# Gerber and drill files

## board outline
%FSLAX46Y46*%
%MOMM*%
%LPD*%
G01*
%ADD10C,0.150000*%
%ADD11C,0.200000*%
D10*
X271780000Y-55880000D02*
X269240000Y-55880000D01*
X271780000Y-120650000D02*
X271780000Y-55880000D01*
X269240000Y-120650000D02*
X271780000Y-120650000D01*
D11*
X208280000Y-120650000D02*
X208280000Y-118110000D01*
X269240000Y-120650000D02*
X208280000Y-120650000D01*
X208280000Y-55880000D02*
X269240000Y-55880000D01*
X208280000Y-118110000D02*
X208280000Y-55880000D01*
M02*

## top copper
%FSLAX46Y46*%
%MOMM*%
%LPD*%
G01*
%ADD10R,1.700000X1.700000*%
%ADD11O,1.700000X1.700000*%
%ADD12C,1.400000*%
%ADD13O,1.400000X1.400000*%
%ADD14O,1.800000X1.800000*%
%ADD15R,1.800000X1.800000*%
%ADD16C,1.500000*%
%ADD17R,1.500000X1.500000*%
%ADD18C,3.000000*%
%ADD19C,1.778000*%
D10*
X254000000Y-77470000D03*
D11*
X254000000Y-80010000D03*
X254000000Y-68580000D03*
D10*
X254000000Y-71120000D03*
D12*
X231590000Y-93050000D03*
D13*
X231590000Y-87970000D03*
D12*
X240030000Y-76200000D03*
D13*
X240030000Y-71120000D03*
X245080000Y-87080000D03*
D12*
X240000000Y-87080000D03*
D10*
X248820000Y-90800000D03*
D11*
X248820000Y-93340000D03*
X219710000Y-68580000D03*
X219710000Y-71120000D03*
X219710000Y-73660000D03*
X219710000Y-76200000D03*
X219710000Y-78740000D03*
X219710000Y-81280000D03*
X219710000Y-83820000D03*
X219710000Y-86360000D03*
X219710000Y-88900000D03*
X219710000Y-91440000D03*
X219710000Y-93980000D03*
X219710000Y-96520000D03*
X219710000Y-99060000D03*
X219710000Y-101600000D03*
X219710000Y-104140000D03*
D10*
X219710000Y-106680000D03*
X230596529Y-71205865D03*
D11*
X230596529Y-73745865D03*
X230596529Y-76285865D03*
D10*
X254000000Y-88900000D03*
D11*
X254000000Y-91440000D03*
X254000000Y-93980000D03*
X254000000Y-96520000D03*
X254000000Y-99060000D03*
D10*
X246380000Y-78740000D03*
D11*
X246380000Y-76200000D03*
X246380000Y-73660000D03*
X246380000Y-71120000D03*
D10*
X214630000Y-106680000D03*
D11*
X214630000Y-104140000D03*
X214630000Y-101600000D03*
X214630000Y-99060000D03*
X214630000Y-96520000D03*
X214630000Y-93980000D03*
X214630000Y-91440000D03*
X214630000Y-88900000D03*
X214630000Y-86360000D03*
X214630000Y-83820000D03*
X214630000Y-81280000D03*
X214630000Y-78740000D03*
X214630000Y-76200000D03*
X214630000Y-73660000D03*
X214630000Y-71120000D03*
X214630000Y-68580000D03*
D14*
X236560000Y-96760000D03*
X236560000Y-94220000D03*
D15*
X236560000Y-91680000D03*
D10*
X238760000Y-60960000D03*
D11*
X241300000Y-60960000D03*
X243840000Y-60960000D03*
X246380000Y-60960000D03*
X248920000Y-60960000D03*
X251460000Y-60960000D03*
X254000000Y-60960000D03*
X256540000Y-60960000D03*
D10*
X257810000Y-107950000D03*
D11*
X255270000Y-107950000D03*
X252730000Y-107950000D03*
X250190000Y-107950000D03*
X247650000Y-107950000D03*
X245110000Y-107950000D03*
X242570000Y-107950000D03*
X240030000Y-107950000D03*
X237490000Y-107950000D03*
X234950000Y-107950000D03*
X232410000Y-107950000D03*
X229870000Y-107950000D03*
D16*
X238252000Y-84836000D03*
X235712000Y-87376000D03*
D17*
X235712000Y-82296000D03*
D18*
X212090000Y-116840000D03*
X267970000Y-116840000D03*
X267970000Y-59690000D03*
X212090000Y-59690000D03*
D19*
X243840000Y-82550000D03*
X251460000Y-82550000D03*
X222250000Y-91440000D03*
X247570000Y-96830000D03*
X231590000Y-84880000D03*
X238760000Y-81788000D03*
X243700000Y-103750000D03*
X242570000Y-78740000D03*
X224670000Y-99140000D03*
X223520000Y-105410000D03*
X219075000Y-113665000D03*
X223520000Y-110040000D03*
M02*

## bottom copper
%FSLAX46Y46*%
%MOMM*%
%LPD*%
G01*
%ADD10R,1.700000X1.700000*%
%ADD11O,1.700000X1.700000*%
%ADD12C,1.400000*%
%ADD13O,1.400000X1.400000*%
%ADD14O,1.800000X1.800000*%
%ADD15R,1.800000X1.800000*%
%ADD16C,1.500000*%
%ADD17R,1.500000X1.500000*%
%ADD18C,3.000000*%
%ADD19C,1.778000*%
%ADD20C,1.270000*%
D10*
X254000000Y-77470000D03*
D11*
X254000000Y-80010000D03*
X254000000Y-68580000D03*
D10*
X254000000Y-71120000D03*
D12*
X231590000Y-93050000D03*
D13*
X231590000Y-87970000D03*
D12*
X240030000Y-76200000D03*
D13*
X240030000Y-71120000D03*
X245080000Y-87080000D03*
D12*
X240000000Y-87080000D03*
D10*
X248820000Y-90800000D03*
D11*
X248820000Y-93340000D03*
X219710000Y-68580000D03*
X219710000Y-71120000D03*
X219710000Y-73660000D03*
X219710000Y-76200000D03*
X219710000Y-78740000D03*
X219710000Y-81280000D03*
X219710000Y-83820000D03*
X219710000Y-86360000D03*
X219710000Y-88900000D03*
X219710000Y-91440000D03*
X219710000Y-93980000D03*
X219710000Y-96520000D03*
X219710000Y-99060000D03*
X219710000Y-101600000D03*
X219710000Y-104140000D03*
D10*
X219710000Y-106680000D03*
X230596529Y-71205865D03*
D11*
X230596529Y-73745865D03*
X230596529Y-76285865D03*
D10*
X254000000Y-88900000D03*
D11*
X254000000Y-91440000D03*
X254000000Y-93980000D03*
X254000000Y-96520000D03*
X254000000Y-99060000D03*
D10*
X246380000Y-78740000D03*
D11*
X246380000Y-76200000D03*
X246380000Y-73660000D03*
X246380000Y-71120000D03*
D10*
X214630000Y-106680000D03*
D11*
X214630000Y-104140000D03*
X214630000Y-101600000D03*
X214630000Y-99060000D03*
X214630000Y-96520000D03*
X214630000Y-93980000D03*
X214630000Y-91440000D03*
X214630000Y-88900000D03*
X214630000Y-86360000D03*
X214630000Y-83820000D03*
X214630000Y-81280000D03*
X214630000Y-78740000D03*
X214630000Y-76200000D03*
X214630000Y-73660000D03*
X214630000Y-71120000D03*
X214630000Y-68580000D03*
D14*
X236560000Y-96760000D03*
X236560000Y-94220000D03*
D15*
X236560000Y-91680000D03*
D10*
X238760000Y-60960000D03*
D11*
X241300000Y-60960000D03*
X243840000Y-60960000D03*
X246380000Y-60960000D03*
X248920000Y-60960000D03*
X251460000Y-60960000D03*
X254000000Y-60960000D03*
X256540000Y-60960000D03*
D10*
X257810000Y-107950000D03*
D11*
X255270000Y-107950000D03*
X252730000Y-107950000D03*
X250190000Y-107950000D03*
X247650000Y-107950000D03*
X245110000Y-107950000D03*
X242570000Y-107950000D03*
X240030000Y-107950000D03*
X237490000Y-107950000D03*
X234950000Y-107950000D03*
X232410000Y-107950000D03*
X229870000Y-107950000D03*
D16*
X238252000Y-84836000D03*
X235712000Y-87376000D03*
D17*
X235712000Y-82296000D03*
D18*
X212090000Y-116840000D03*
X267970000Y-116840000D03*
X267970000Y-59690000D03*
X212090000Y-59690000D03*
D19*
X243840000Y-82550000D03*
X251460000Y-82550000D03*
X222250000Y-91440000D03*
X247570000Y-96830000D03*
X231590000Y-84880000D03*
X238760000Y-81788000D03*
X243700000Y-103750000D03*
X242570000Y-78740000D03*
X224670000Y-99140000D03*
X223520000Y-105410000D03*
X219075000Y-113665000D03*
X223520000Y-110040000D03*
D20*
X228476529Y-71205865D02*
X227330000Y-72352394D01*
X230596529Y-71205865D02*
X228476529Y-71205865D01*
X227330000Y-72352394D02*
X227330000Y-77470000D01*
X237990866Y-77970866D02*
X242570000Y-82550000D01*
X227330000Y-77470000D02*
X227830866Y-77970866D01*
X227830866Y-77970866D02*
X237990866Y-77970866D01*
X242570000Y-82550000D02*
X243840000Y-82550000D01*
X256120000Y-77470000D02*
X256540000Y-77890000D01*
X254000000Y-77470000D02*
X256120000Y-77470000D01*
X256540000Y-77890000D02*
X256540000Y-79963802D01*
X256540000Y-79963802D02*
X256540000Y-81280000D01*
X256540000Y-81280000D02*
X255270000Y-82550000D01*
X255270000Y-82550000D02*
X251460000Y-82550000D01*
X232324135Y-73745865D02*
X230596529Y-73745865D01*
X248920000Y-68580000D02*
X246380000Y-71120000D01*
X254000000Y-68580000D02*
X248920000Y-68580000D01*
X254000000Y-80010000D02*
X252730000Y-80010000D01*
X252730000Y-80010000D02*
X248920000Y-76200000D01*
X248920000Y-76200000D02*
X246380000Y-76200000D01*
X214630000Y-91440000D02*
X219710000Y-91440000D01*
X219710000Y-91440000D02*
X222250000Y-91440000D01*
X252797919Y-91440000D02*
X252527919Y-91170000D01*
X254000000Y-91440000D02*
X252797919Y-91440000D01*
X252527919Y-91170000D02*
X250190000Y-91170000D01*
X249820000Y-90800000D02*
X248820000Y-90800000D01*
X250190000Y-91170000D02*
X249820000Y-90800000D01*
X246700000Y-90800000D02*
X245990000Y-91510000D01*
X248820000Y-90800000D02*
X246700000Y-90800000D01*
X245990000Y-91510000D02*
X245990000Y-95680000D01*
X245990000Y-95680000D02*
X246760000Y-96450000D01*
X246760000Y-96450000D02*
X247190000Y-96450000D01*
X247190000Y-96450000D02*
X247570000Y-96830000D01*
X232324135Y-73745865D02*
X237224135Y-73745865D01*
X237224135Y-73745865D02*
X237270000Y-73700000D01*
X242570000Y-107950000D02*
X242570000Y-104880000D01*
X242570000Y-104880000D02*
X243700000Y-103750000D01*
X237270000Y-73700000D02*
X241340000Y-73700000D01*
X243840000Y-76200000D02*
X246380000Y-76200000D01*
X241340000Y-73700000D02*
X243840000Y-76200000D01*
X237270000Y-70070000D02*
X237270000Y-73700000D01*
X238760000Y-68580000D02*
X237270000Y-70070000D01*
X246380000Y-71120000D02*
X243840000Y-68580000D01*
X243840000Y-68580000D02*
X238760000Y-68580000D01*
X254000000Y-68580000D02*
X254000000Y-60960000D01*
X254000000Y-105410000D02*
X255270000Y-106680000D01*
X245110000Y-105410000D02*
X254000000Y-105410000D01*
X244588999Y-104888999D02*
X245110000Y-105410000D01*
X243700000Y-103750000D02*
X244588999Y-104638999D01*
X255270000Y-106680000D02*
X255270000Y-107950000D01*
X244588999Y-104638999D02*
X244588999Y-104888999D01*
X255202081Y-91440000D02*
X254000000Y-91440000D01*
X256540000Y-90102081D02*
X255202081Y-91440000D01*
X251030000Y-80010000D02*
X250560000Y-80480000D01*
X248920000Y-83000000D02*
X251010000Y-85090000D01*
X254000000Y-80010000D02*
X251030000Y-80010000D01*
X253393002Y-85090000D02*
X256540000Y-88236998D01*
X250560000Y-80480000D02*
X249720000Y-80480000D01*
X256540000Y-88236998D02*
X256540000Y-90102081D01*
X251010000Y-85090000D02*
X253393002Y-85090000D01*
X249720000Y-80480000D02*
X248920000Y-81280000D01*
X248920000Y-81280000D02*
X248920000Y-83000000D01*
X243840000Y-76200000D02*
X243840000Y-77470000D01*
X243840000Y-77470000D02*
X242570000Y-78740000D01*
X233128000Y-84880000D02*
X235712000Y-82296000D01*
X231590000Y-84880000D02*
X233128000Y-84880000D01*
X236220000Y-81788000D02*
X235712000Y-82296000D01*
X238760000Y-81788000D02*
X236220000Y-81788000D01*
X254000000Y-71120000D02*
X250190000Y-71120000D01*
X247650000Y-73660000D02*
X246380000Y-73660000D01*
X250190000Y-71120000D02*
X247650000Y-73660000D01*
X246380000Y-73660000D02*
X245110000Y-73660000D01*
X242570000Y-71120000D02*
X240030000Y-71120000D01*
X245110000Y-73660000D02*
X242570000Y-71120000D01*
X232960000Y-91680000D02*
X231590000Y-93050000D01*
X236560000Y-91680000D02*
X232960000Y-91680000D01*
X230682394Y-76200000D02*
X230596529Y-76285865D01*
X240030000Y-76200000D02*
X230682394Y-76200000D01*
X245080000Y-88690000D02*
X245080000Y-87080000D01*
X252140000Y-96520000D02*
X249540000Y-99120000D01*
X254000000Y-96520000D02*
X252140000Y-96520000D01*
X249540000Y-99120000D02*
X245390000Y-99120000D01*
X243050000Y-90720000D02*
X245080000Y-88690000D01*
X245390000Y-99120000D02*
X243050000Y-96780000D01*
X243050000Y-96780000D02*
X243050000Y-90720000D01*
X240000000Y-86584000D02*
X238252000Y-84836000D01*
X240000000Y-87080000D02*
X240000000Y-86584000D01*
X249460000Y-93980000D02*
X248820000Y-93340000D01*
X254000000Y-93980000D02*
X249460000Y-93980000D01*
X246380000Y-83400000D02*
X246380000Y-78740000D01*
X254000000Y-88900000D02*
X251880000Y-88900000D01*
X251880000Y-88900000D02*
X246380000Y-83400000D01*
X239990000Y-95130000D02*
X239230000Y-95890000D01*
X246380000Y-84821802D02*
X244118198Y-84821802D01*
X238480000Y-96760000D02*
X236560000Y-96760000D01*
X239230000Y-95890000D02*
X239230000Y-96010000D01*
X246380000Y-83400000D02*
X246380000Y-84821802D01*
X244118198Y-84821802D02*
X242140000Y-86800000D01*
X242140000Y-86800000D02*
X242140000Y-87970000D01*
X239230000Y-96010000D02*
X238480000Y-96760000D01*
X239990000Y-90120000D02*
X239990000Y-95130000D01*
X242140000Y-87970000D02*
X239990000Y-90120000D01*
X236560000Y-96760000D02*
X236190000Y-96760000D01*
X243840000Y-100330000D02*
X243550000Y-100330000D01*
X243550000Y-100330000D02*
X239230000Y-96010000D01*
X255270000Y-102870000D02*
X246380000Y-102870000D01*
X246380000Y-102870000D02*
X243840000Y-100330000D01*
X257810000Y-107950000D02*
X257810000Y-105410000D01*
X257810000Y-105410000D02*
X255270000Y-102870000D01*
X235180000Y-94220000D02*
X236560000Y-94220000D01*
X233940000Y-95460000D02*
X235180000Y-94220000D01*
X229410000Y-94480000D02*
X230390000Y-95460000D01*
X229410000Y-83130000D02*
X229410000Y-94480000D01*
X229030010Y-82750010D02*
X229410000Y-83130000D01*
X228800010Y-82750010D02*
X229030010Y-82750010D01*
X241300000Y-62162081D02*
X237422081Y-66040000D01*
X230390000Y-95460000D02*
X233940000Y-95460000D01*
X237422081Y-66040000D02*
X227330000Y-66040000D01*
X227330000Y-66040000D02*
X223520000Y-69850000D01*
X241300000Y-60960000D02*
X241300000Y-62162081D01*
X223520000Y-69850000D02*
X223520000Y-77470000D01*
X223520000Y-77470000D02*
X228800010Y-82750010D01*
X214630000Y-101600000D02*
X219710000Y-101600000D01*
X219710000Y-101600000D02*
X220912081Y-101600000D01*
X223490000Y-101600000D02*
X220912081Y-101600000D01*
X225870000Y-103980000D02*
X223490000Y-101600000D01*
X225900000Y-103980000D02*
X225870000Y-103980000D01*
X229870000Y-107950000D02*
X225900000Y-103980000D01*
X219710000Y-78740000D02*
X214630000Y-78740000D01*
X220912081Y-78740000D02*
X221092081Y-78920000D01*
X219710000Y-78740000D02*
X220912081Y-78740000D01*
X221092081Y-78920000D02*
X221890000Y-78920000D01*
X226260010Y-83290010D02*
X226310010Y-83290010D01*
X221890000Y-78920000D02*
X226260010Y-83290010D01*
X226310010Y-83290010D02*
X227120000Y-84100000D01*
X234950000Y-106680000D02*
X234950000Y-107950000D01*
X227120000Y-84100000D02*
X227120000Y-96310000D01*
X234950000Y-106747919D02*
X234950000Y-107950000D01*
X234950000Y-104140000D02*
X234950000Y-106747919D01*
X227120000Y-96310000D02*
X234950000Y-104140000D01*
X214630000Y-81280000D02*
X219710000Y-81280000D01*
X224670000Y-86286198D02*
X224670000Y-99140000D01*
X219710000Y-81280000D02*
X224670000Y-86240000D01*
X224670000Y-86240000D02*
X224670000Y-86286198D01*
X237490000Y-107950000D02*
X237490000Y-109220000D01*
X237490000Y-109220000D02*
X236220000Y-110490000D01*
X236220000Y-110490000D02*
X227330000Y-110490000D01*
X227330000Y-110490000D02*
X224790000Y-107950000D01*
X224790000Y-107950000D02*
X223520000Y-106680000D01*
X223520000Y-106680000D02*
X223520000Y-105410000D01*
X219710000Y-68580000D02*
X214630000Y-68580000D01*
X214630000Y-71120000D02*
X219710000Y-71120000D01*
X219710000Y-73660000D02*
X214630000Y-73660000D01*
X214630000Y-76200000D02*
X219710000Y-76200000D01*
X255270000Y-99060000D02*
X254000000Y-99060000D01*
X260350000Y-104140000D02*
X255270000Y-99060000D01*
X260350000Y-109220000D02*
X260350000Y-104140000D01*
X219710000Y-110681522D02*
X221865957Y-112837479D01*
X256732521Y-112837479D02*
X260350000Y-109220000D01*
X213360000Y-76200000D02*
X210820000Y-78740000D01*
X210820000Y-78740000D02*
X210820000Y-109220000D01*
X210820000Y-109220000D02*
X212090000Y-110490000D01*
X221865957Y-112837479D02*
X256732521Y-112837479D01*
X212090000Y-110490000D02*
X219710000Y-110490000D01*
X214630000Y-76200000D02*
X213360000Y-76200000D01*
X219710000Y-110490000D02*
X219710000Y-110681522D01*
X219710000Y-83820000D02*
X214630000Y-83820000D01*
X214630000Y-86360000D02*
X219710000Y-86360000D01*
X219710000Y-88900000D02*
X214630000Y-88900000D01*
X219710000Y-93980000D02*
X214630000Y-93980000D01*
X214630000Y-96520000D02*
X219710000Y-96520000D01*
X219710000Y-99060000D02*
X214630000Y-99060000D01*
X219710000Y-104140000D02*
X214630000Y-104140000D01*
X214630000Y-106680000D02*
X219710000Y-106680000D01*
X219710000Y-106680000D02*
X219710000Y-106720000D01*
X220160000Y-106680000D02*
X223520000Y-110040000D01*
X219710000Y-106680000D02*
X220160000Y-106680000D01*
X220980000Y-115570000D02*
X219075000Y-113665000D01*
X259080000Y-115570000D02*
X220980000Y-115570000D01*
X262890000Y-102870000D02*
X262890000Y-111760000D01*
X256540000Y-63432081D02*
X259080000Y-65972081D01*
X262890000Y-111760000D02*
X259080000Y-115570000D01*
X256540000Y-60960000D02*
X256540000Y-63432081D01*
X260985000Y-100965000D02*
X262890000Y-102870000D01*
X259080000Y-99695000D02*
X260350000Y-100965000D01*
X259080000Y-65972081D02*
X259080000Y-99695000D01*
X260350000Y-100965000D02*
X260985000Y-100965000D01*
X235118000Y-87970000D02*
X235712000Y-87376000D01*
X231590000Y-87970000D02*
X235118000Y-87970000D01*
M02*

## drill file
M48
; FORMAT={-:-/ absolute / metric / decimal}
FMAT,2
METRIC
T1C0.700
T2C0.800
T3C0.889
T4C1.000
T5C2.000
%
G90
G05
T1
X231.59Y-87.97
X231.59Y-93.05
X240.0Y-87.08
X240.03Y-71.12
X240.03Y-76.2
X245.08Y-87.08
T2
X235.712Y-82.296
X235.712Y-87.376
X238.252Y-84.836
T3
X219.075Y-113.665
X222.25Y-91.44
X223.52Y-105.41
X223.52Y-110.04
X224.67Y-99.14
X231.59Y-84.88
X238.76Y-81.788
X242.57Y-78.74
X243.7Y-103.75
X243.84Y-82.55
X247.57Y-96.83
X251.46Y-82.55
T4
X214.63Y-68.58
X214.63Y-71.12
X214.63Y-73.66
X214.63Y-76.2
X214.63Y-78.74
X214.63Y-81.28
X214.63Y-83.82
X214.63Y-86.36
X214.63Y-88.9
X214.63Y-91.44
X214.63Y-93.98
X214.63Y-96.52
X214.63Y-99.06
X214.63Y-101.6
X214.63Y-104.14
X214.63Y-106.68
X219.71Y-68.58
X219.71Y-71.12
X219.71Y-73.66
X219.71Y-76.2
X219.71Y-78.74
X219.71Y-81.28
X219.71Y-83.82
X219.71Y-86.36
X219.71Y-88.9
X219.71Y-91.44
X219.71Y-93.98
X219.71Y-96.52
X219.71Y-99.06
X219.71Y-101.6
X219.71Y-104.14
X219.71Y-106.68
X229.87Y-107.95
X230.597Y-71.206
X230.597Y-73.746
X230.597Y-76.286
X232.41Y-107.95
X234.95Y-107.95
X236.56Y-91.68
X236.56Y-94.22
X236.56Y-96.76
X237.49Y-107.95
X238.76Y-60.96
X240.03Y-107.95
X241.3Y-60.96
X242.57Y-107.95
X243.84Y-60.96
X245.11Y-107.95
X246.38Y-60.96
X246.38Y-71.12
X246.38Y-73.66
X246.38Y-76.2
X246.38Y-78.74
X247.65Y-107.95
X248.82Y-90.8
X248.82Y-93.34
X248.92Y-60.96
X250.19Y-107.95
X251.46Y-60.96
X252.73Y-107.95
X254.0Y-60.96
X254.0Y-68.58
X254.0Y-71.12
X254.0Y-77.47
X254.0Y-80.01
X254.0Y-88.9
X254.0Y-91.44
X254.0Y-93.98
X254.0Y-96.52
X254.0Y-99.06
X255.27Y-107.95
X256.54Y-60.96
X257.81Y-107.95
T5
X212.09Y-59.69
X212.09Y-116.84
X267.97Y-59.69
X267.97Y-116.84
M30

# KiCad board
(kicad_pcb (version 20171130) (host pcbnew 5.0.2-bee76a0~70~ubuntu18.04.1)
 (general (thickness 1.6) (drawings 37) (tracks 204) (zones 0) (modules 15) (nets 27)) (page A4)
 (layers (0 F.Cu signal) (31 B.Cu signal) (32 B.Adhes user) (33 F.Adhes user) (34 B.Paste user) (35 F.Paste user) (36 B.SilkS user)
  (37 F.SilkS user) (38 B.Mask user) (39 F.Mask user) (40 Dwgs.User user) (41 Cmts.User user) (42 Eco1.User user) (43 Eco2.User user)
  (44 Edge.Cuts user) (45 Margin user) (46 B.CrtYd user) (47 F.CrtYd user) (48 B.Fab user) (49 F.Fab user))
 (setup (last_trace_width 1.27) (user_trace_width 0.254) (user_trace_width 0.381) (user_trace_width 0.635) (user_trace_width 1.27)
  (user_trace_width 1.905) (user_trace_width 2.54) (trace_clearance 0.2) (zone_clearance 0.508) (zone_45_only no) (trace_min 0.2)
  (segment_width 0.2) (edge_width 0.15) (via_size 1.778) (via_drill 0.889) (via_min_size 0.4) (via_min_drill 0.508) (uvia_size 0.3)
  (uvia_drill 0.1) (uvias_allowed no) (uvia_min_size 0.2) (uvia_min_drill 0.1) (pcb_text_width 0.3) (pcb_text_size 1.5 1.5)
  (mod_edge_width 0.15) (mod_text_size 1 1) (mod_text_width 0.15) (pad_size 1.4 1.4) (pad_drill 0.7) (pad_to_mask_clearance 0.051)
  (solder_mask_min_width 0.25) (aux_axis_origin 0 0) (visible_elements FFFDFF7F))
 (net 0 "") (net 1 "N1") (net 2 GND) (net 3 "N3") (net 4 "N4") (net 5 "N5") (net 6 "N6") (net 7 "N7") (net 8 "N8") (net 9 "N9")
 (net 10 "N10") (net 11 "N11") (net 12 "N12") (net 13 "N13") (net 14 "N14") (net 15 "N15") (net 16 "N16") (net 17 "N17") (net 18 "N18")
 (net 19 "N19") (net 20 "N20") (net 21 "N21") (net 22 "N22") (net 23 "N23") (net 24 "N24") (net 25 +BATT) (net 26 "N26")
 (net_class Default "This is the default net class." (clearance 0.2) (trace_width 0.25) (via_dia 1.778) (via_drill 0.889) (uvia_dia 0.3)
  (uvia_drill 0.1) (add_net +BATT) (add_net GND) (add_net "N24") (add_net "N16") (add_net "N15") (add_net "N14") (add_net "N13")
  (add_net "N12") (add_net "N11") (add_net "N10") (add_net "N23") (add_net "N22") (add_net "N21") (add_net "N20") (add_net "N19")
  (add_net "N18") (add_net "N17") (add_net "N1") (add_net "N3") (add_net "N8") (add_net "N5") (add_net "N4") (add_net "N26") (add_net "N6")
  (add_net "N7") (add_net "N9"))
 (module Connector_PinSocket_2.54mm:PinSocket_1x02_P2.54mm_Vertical (layer F.Cu) (at 254 77.47)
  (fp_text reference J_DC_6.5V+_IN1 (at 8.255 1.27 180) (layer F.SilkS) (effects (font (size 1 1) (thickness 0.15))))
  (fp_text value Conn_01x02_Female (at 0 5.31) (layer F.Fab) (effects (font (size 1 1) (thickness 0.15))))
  (pad 1 thru_hole rect (at 0 0) (size 1.7 1.7) (drill 1) (layers *.Cu *.Mask) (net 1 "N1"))
  (pad 2 thru_hole oval (at 0 2.54) (size 1.7 1.7) (drill 1) (layers *.Cu *.Mask) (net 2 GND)))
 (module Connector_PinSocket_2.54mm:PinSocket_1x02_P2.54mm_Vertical (layer F.Cu) (at 254 71.12 180)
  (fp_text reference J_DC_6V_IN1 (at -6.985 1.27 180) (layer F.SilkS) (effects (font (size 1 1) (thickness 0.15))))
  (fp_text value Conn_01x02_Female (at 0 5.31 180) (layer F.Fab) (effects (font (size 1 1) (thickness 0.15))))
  (pad 2 thru_hole oval (at 0 2.54 180) (size 1.7 1.7) (drill 1) (layers *.Cu *.Mask) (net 2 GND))
  (pad 1 thru_hole rect (at 0 0 180) (size 1.7 1.7) (drill 1) (layers *.Cu *.Mask) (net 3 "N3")))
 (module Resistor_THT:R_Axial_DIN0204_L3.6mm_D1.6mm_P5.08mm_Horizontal (layer F.Cu) (at 231.59 93.05 90)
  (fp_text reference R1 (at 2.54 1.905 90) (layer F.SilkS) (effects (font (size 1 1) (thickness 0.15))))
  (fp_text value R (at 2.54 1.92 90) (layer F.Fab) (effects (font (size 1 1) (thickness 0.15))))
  (pad 1 thru_hole circle (at 0 0 90) (size 1.4 1.4) (drill 0.7) (layers *.Cu *.Mask) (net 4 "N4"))
  (pad 2 thru_hole oval (at 5.08 0 90) (size 1.4 1.4) (drill 0.7) (layers *.Cu *.Mask) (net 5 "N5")))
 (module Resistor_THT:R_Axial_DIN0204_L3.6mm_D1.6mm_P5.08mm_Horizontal (layer F.Cu) (at 240.03 76.2 90)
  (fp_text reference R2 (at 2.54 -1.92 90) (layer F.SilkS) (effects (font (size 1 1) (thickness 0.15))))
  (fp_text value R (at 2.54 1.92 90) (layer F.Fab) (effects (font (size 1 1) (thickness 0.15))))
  (pad 1 thru_hole circle (at 0 0 90) (size 1.4 1.4) (drill 0.7) (layers *.Cu *.Mask) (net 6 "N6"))
  (pad 2 thru_hole oval (at 5.08 0 90) (size 1.4 1.4) (drill 0.7) (layers *.Cu *.Mask) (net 3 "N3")))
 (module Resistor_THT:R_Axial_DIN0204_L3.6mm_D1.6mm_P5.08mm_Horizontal (layer F.Cu) (at 240 87.08)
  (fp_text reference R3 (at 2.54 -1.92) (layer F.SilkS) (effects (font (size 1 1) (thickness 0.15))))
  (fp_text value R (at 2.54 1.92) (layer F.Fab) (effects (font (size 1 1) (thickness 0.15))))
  (pad 2 thru_hole oval (at 5.08 0) (size 1.4 1.4) (drill 0.7) (layers *.Cu *.Mask) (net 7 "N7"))
  (pad 1 thru_hole circle (at 0 0) (size 1.4 1.4) (drill 0.7) (layers *.Cu *.Mask) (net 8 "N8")))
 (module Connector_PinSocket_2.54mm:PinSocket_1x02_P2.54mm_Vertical (layer F.Cu) (at 248.82 90.8)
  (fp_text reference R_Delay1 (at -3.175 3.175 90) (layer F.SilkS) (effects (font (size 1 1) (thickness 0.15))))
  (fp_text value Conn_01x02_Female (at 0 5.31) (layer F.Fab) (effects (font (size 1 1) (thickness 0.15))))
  (pad 1 thru_hole rect (at 0 0) (size 1.7 1.7) (drill 1) (layers *.Cu *.Mask) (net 2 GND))
  (pad 2 thru_hole oval (at 0 2.54) (size 1.7 1.7) (drill 1) (layers *.Cu *.Mask) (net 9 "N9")))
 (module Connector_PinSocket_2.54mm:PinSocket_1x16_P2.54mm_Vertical (layer F.Cu) (at 219.71 106.68 180)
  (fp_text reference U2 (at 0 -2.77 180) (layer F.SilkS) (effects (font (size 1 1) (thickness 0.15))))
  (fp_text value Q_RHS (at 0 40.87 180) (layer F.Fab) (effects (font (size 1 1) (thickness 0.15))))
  (pad 16 thru_hole oval (at 0 38.1 180) (size 1.7 1.7) (drill 1) (layers *.Cu *.Mask) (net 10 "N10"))
  (pad 15 thru_hole oval (at 0 35.56 180) (size 1.7 1.7) (drill 1) (layers *.Cu *.Mask) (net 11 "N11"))
  (pad 14 thru_hole oval (at 0 33.02 180) (size 1.7 1.7) (drill 1) (layers *.Cu *.Mask) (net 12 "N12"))
  (pad 13 thru_hole oval (at 0 30.48 180) (size 1.7 1.7) (drill 1) (layers *.Cu *.Mask) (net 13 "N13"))
  (pad 12 thru_hole oval (at 0 27.94 180) (size 1.7 1.7) (drill 1) (layers *.Cu *.Mask) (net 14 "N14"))
  (pad 11 thru_hole oval (at 0 25.4 180) (size 1.7 1.7) (drill 1) (layers *.Cu *.Mask) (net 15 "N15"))
  (pad 10 thru_hole oval (at 0 22.86 180) (size 1.7 1.7) (drill 1) (layers *.Cu *.Mask) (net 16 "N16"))
  (pad 9 thru_hole oval (at 0 20.32 180) (size 1.7 1.7) (drill 1) (layers *.Cu *.Mask) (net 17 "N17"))
  (pad 8 thru_hole oval (at 0 17.78 180) (size 1.7 1.7) (drill 1) (layers *.Cu *.Mask) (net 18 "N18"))
  (pad 7 thru_hole oval (at 0 15.24 180) (size 1.7 1.7) (drill 1) (layers *.Cu *.Mask) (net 2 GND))
  (pad 6 thru_hole oval (at 0 12.7 180) (size 1.7 1.7) (drill 1) (layers *.Cu *.Mask) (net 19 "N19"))
  (pad 5 thru_hole oval (at 0 10.16 180) (size 1.7 1.7) (drill 1) (layers *.Cu *.Mask) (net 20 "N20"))
  (pad 4 thru_hole oval (at 0 7.62 180) (size 1.7 1.7) (drill 1) (layers *.Cu *.Mask) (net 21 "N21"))
  (pad 3 thru_hole oval (at 0 5.08 180) (size 1.7 1.7) (drill 1) (layers *.Cu *.Mask) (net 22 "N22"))
  (pad 2 thru_hole oval (at 0 2.54 180) (size 1.7 1.7) (drill 1) (layers *.Cu *.Mask) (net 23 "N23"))
  (pad 1 thru_hole rect (at 0 0 180) (size 1.7 1.7) (drill 1) (layers *.Cu *.Mask) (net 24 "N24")))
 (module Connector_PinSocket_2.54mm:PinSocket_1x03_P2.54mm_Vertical (layer F.Cu) (at 230.596529 71.205865)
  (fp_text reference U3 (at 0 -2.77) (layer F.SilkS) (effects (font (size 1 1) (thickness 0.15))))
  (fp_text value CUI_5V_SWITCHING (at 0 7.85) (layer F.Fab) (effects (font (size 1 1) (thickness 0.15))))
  (pad 1 thru_hole rect (at 0 0) (size 1.7 1.7) (drill 1) (layers *.Cu *.Mask) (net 1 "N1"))
  (pad 2 thru_hole oval (at 0 2.54) (size 1.7 1.7) (drill 1) (layers *.Cu *.Mask) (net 2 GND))
  (pad 3 thru_hole oval (at 0 5.08) (size 1.7 1.7) (drill 1) (layers *.Cu *.Mask) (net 6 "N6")))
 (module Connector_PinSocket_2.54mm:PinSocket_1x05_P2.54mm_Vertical (layer F.Cu) (at 254 88.9)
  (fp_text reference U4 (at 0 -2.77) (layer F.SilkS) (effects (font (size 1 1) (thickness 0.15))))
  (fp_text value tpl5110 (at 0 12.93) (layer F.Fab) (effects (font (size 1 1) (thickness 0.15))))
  (pad 1 thru_hole rect (at 0 0) (size 1.7 1.7) (drill 1) (layers *.Cu *.Mask) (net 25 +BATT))
  (pad 2 thru_hole oval (at 0 2.54) (size 1.7 1.7) (drill 1) (layers *.Cu *.Mask) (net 2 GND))
  (pad 3 thru_hole oval (at 0 5.08) (size 1.7 1.7) (drill 1) (layers *.Cu *.Mask) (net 9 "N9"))
  (pad 4 thru_hole oval (at 0 7.62) (size 1.7 1.7) (drill 1) (layers *.Cu *.Mask) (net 7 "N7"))
  (pad 5 thru_hole oval (at 0 10.16) (size 1.7 1.7) (drill 1) (layers *.Cu *.Mask) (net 13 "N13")))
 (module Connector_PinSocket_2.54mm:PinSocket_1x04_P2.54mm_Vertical (layer F.Cu) (at 246.38 78.74 180)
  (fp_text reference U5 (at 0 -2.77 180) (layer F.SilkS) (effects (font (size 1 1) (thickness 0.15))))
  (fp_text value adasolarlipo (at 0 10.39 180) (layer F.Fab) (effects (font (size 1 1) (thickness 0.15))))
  (pad 1 thru_hole rect (at 0 0 180) (size 1.7 1.7) (drill 1) (layers *.Cu *.Mask) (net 25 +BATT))
  (pad 2 thru_hole oval (at 0 2.54 180) (size 1.7 1.7) (drill 1) (layers *.Cu *.Mask) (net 2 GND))
  (pad 3 thru_hole oval (at 0 5.08 180) (size 1.7 1.7) (drill 1) (layers *.Cu *.Mask) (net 3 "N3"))
  (pad 4 thru_hole oval (at 0 7.62 180) (size 1.7 1.7) (drill 1) (layers *.Cu *.Mask) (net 2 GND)))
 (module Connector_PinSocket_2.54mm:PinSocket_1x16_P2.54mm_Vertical (layer F.Cu) (at 214.63 106.68 180)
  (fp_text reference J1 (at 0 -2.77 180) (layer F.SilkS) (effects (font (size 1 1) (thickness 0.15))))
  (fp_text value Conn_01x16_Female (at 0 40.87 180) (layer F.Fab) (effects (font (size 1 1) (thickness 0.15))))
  (pad 1 thru_hole rect (at 0 0 180) (size 1.7 1.7) (drill 1) (layers *.Cu *.Mask) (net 24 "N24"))
  (pad 2 thru_hole oval (at 0 2.54 180) (size 1.7 1.7) (drill 1) (layers *.Cu *.Mask) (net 23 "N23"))
  (pad 3 thru_hole oval (at 0 5.08 180) (size 1.7 1.7) (drill 1) (layers *.Cu *.Mask) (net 22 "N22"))
  (pad 4 thru_hole oval (at 0 7.62 180) (size 1.7 1.7) (drill 1) (layers *.Cu *.Mask) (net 21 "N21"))
  (pad 5 thru_hole oval (at 0 10.16 180) (size 1.7 1.7) (drill 1) (layers *.Cu *.Mask) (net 20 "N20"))
  (pad 6 thru_hole oval (at 0 12.7 180) (size 1.7 1.7) (drill 1) (layers *.Cu *.Mask) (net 19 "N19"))
  (pad 7 thru_hole oval (at 0 15.24 180) (size 1.7 1.7) (drill 1) (layers *.Cu *.Mask) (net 2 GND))
  (pad 8 thru_hole oval (at 0 17.78 180) (size 1.7 1.7) (drill 1) (layers *.Cu *.Mask) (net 18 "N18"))
  (pad 9 thru_hole oval (at 0 20.32 180) (size 1.7 1.7) (drill 1) (layers *.Cu *.Mask) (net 17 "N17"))
  (pad 10 thru_hole oval (at 0 22.86 180) (size 1.7 1.7) (drill 1) (layers *.Cu *.Mask) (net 16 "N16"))
  (pad 11 thru_hole oval (at 0 25.4 180) (size 1.7 1.7) (drill 1) (layers *.Cu *.Mask) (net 15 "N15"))
  (pad 12 thru_hole oval (at 0 27.94 180) (size 1.7 1.7) (drill 1) (layers *.Cu *.Mask) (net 14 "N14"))
  (pad 13 thru_hole oval (at 0 30.48 180) (size 1.7 1.7) (drill 1) (layers *.Cu *.Mask) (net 13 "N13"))
  (pad 14 thru_hole oval (at 0 33.02 180) (size 1.7 1.7) (drill 1) (layers *.Cu *.Mask) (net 12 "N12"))
  (pad 15 thru_hole oval (at 0 35.56 180) (size 1.7 1.7) (drill 1) (layers *.Cu *.Mask) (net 11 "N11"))
  (pad 16 thru_hole oval (at 0 38.1 180) (size 1.7 1.7) (drill 1) (layers *.Cu *.Mask) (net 10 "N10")))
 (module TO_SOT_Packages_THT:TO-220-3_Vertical (layer F.Cu) (at 236.56 91.68 270)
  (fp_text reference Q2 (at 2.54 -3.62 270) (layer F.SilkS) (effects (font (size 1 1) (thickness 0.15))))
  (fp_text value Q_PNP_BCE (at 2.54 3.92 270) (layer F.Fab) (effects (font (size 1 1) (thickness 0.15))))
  (pad 3 thru_hole oval (at 5.08 0 270) (size 1.8 1.8) (drill 1) (layers *.Cu *.Mask) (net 25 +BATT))
  (pad 2 thru_hole oval (at 2.54 0 270) (size 1.8 1.8) (drill 1) (layers *.Cu *.Mask) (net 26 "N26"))
  (pad 1 thru_hole rect (at 0 0 270) (size 1.8 1.8) (drill 1) (layers *.Cu *.Mask) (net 4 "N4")))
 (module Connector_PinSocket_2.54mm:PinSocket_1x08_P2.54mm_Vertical (layer F.Cu) (at 238.76 60.96 90)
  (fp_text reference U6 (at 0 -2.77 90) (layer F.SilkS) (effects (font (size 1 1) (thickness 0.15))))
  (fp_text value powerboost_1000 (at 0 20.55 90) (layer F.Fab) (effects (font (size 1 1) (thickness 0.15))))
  (pad 1 thru_hole rect (at 0 0 90) (size 1.7 1.7) (drill 1) (layers *.Cu *.Mask))
  (pad 2 thru_hole oval (at 0 2.54 90) (size 1.7 1.7) (drill 1) (layers *.Cu *.Mask) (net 26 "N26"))
  (pad 3 thru_hole oval (at 0 5.08 90) (size 1.7 1.7) (drill 1) (layers *.Cu *.Mask))
  (pad 4 thru_hole oval (at 0 7.62 90) (size 1.7 1.7) (drill 1) (layers *.Cu *.Mask))
  (pad 5 thru_hole oval (at 0 10.16 90) (size 1.7 1.7) (drill 1) (layers *.Cu *.Mask))
  (pad 6 thru_hole oval (at 0 12.7 90) (size 1.7 1.7) (drill 1) (layers *.Cu *.Mask))
  (pad 7 thru_hole oval (at 0 15.24 90) (size 1.7 1.7) (drill 1) (layers *.Cu *.Mask) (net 2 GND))
  (pad 8 thru_hole oval (at 0 17.78 90) (size 1.7 1.7) (drill 1) (layers *.Cu *.Mask) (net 24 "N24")))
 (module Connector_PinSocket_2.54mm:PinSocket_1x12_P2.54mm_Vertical (layer F.Cu) (at 257.81 107.95 270)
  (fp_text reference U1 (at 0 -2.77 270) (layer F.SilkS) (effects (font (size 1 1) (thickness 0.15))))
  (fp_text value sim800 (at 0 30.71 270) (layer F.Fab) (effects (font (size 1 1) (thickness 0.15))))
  (pad 1 thru_hole rect (at 0 0 270) (size 1.7 1.7) (drill 1) (layers *.Cu *.Mask) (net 25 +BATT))
  (pad 2 thru_hole oval (at 0 2.54 270) (size 1.7 1.7) (drill 1) (layers *.Cu *.Mask) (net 2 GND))
  (pad 3 thru_hole oval (at 0 5.08 270) (size 1.7 1.7) (drill 1) (layers *.Cu *.Mask))
  (pad 4 thru_hole oval (at 0 7.62 270) (size 1.7 1.7) (drill 1) (layers *.Cu *.Mask))
  (pad 5 thru_hole oval (at 0 10.16 270) (size 1.7 1.7) (drill 1) (layers *.Cu *.Mask))
  (pad 6 thru_hole oval (at 0 12.7 270) (size 1.7 1.7) (drill 1) (layers *.Cu *.Mask))
  (pad 7 thru_hole oval (at 0 15.24 270) (size 1.7 1.7) (drill 1) (layers *.Cu *.Mask) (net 2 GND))
  (pad 8 thru_hole oval (at 0 17.78 270) (size 1.7 1.7) (drill 1) (layers *.Cu *.Mask))
  (pad 9 thru_hole oval (at 0 20.32 270) (size 1.7 1.7) (drill 1) (layers *.Cu *.Mask) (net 15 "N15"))
  (pad 10 thru_hole oval (at 0 22.86 270) (size 1.7 1.7) (drill 1) (layers *.Cu *.Mask) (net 14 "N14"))
  (pad 11 thru_hole oval (at 0 25.4 270) (size 1.7 1.7) (drill 1) (layers *.Cu *.Mask))
  (pad 12 thru_hole oval (at 0 27.94 270) (size 1.7 1.7) (drill 1) (layers *.Cu *.Mask) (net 22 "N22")))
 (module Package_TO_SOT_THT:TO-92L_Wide (layer F.Cu) (at 235.712 82.296 270)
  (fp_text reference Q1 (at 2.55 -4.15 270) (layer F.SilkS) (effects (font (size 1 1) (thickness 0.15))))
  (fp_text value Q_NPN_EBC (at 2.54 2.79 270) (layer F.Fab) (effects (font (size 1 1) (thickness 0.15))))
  (pad 2 thru_hole circle (at 2.54 -2.54) (size 1.5 1.5) (drill 0.8) (layers *.Cu *.Mask) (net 8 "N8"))
  (pad 3 thru_hole circle (at 5.08 0) (size 1.5 1.5) (drill 0.8) (layers *.Cu *.Mask) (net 5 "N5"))
  (pad 1 thru_hole rect (at 0 0) (size 1.5 1.5) (drill 0.8) (layers *.Cu *.Mask) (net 2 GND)))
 (gr_line (start 271.78 55.88) (end 269.24 55.88) (layer Edge.Cuts) (width 0.15))
 (gr_line (start 271.78 120.65) (end 271.78 55.88) (layer Edge.Cuts) (width 0.15))
 (gr_line (start 269.24 120.65) (end 271.78 120.65) (layer Edge.Cuts) (width 0.15))
 (gr_line (start 208.28 120.65) (end 208.28 118.11) (layer Edge.Cuts) (width 0.2))
 (gr_line (start 269.24 120.65) (end 208.28 120.65) (layer Edge.Cuts) (width 0.2))
 (gr_line (start 208.28 55.88) (end 269.24 55.88) (layer Edge.Cuts) (width 0.2))
 (gr_line (start 208.28 118.11) (end 208.28 55.88) (layer Edge.Cuts) (width 0.2))
 (via (at 212.09 116.84) (size 3) (drill 2) (layers F.Cu B.Cu) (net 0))
 (via (at 267.97 116.84) (size 3) (drill 2) (layers F.Cu B.Cu) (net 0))
 (via (at 267.97 59.69) (size 3) (drill 2) (layers F.Cu B.Cu) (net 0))
 (via (at 212.09 59.69) (size 3) (drill 2) (layers F.Cu B.Cu) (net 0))
 (segment (start 228.476529 71.205865) (end 227.33 72.352394) (width 1.27) (layer B.Cu) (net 1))
 (segment (start 230.596529 71.205865) (end 228.476529 71.205865) (width 1.27) (layer B.Cu) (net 1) (status 10))
 (segment (start 227.33 72.352394) (end 227.33 77.47) (width 1.27) (layer B.Cu) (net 1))
 (segment (start 237.990866 77.970866) (end 242.57 82.55) (width 1.27) (layer B.Cu) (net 1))
 (segment (start 227.33 77.47) (end 227.830866 77.970866) (width 1.27) (layer B.Cu) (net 1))
 (segment (start 227.830866 77.970866) (end 237.990866 77.970866) (width 1.27) (layer B.Cu) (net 1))
 (via (at 243.84 82.55) (size 1.778) (drill 0.889) (layers F.Cu B.Cu) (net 1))
 (segment (start 242.57 82.55) (end 243.84 82.55) (width 1.27) (layer B.Cu) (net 1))
 (segment (start 256.12 77.47) (end 256.54 77.89) (width 1.27) (layer B.Cu) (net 1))
 (segment (start 254 77.47) (end 256.12 77.47) (width 1.27) (layer B.Cu) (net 1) (status 10))
 (segment (start 256.54 77.89) (end 256.54 79.963802) (width 1.27) (layer B.Cu) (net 1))
 (segment (start 256.54 79.963802) (end 256.54 81.28) (width 1.27) (layer B.Cu) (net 1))
 (segment (start 256.54 81.28) (end 255.27 82.55) (width 1.27) (layer B.Cu) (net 1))
 (via (at 251.46 82.55) (size 1.778) (drill 0.889) (layers F.Cu B.Cu) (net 1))
 (segment (start 255.27 82.55) (end 251.46 82.55) (width 1.27) (layer B.Cu) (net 1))
 (segment (start 232.324135 73.745865) (end 230.596529 73.745865) (width 1.27) (layer B.Cu) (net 2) (status 20))
 (segment (start 248.92 68.58) (end 246.38 71.12) (width 1.27) (layer B.Cu) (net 2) (status 20))
 (segment (start 254 68.58) (end 248.92 68.58) (width 1.27) (layer B.Cu) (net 2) (status 10))
 (segment (start 254 80.01) (end 252.73 80.01) (width 1.27) (layer B.Cu) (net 2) (status 10))
 (segment (start 252.73 80.01) (end 248.92 76.2) (width 1.27) (layer B.Cu) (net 2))
 (segment (start 248.92 76.2) (end 246.38 76.2) (width 1.27) (layer B.Cu) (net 2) (status 20))
 (segment (start 214.63 91.44) (end 219.71 91.44) (width 1.27) (layer B.Cu) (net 2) (status 30))
 (via (at 222.25 91.44) (size 1.778) (drill 0.889) (layers F.Cu B.Cu) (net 2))
 (segment (start 219.71 91.44) (end 222.25 91.44) (width 1.27) (layer B.Cu) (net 2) (status 10))
 (segment (start 252.797919 91.44) (end 252.527919 91.17) (width 1.27) (layer B.Cu) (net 2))
 (segment (start 254 91.44) (end 252.797919 91.44) (width 1.27) (layer B.Cu) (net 2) (status 10))
 (segment (start 252.527919 91.17) (end 250.19 91.17) (width 1.27) (layer B.Cu) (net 2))
 (segment (start 249.82 90.8) (end 248.82 90.8) (width 1.27) (layer B.Cu) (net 2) (status 20))
 (segment (start 250.19 91.17) (end 249.82 90.8) (width 1.27) (layer B.Cu) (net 2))
 (segment (start 246.7 90.8) (end 245.99 91.51) (width 1.27) (layer B.Cu) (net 2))
 (segment (start 248.82 90.8) (end 246.7 90.8) (width 1.27) (layer B.Cu) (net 2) (status 10))
 (segment (start 245.99 91.51) (end 245.99 95.68) (width 1.27) (layer B.Cu) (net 2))
 (segment (start 245.99 95.68) (end 246.76 96.45) (width 1.27) (layer B.Cu) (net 2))
 (via (at 247.57 96.83) (size 1.778) (drill 0.889) (layers F.Cu B.Cu) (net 2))
 (segment (start 246.76 96.45) (end 247.19 96.45) (width 1.27) (layer B.Cu) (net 2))
 (segment (start 247.19 96.45) (end 247.57 96.83) (width 1.27) (layer B.Cu) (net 2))
 (via (at 231.59 84.88) (size 1.778) (drill 0.889) (layers F.Cu B.Cu) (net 2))
 (via (at 238.76 81.788) (size 1.778) (drill 0.889) (layers F.Cu B.Cu) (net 2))
 (segment (start 232.324135 73.745865) (end 237.224135 73.745865) (width 1.27) (layer B.Cu) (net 2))
 (segment (start 237.224135 73.745865) (end 237.27 73.7) (width 1.27) (layer B.Cu) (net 2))
 (via (at 243.7 103.75) (size 1.778) (drill 0.889) (layers F.Cu B.Cu) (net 2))
 (segment (start 242.57 107.95) (end 242.57 104.88) (width 1.27) (layer B.Cu) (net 2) (status 10))
 (segment (start 242.57 104.88) (end 243.7 103.75) (width 1.27) (layer B.Cu) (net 2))
 (segment (start 237.27 73.7) (end 241.34 73.7) (width 1.27) (layer B.Cu) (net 2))
 (segment (start 243.84 76.2) (end 246.38 76.2) (width 1.27) (layer B.Cu) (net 2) (status 20))
 (segment (start 241.34 73.7) (end 243.84 76.2) (width 1.27) (layer B.Cu) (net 2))
 (segment (start 237.27 70.07) (end 237.27 73.7) (width 1.27) (layer B.Cu) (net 2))
 (segment (start 238.76 68.58) (end 237.27 70.07) (width 1.27) (layer B.Cu) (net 2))
 (segment (start 246.38 71.12) (end 243.84 68.58) (width 1.27) (layer B.Cu) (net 2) (status 10))
 (segment (start 243.84 68.58) (end 238.76 68.58) (width 1.27) (layer B.Cu) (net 2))
 (segment (start 254 68.58) (end 254 60.96) (width 1.27) (layer B.Cu) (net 2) (status 30))
 (segment (start 254 105.41) (end 255.27 106.68) (width 1.27) (layer B.Cu) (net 2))
 (segment (start 245.11 105.41) (end 254 105.41) (width 1.27) (layer B.Cu) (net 2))
 (segment (start 244.588999 104.888999) (end 245.11 105.41) (width 1.27) (layer B.Cu) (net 2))
 (segment (start 243.7 103.75) (end 244.588999 104.638999) (width 1.27) (layer B.Cu) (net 2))
 (segment (start 255.27 106.68) (end 255.27 107.95) (width 1.27) (layer B.Cu) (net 2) (status 20))
 (segment (start 244.588999 104.638999) (end 244.588999 104.888999) (width 1.27) (layer B.Cu) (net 2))
 (segment (start 255.202081 91.44) (end 254 91.44) (width 1.27) (layer B.Cu) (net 2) (status 20))
 (segment (start 256.54 90.102081) (end 255.202081 91.44) (width 1.27) (layer B.Cu) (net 2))
 (segment (start 251.03 80.01) (end 250.56 80.48) (width 1.27) (layer B.Cu) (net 2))
 (segment (start 248.92 83) (end 251.01 85.09) (width 1.27) (layer B.Cu) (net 2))
 (segment (start 254 80.01) (end 251.03 80.01) (width 1.27) (layer B.Cu) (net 2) (status 10))
 (segment (start 253.393002 85.09) (end 256.54 88.236998) (width 1.27) (layer B.Cu) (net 2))
 (segment (start 250.56 80.48) (end 249.72 80.48) (width 1.27) (layer B.Cu) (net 2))
 (segment (start 256.54 88.236998) (end 256.54 90.102081) (width 1.27) (layer B.Cu) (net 2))
 (segment (start 251.01 85.09) (end 253.393002 85.09) (width 1.27) (layer B.Cu) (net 2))
 (segment (start 249.72 80.48) (end 248.92 81.28) (width 1.27) (layer B.Cu) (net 2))
 (segment (start 248.92 81.28) (end 248.92 83) (width 1.27) (layer B.Cu) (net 2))
 (via (at 242.57 78.74) (size 1.778) (drill 0.889) (layers F.Cu B.Cu) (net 2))
 (segment (start 243.84 76.2) (end 243.84 77.47) (width 1.27) (layer B.Cu) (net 2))
 (segment (start 243.84 77.47) (end 242.57 78.74) (width 1.27) (layer B.Cu) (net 2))
 (segment (start 233.128 84.88) (end 235.712 82.296) (width 1.27) (layer B.Cu) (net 2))
 (segment (start 231.59 84.88) (end 233.128 84.88) (width 1.27) (layer B.Cu) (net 2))
 (segment (start 236.22 81.788) (end 235.712 82.296) (width 1.27) (layer B.Cu) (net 2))
 (segment (start 238.76 81.788) (end 236.22 81.788) (width 1.27) (layer B.Cu) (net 2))
 (segment (start 254 71.12) (end 250.19 71.12) (width 1.27) (layer B.Cu) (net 3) (status 10))
 (segment (start 247.65 73.66) (end 246.38 73.66) (width 1.27) (layer B.Cu) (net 3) (status 20))
 (segment (start 250.19 71.12) (end 247.65 73.66) (width 1.27) (layer B.Cu) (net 3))
 (segment (start 246.38 73.66) (end 245.11 73.66) (width 1.27) (layer B.Cu) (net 3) (status 10))
 (segment (start 242.57 71.12) (end 240.03 71.12) (width 1.27) (layer B.Cu) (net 3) (status 20))
 (segment (start 245.11 73.66) (end 242.57 71.12) (width 1.27) (layer B.Cu) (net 3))
 (segment (start 232.96 91.68) (end 231.59 93.05) (width 1.27) (layer B.Cu) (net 4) (status 20))
 (segment (start 236.56 91.68) (end 232.96 91.68) (width 1.27) (layer B.Cu) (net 4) (status 10))
 (segment (start 230.682394 76.2) (end 230.596529 76.285865) (width 1.27) (layer B.Cu) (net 6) (status 30))
 (segment (start 240.03 76.2) (end 230.682394 76.2) (width 1.27) (layer B.Cu) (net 6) (status 30))
 (segment (start 245.08 88.69) (end 245.08 87.08) (width 1.27) (layer B.Cu) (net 7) (status 20))
 (segment (start 252.14 96.52) (end 249.54 99.12) (width 1.27) (layer B.Cu) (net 7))
 (segment (start 254 96.52) (end 252.14 96.52) (width 1.27) (layer B.Cu) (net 7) (status 10))
 (segment (start 249.54 99.12) (end 245.39 99.12) (width 1.27) (layer B.Cu) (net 7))
 (segment (start 243.05 90.72) (end 245.08 88.69) (width 1.27) (layer B.Cu) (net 7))
 (segment (start 245.39 99.12) (end 243.05 96.78) (width 1.27) (layer B.Cu) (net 7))
 (segment (start 243.05 96.78) (end 243.05 90.72) (width 1.27) (layer B.Cu) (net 7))
 (segment (start 240 86.584) (end 238.252 84.836) (width 1.27) (layer B.Cu) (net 8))
 (segment (start 240 87.08) (end 240 86.584) (width 1.27) (layer B.Cu) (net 8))
 (segment (start 249.46 93.98) (end 248.82 93.34) (width 1.27) (layer B.Cu) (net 9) (status 30))
 (segment (start 254 93.98) (end 249.46 93.98) (width 1.27) (layer B.Cu) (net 9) (status 30))
 (segment (start 246.38 83.4) (end 246.38 78.74) (width 1.27) (layer B.Cu) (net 25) (status 20))
 (segment (start 254 88.9) (end 251.88 88.9) (width 1.27) (layer B.Cu) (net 25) (status 10))
 (segment (start 251.88 88.9) (end 246.38 83.4) (width 1.27) (layer B.Cu) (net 25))
 (segment (start 239.99 95.13) (end 239.23 95.89) (width 1.27) (layer B.Cu) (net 25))
 (segment (start 246.38 84.821802) (end 244.118198 84.821802) (width 1.27) (layer B.Cu) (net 25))
 (segment (start 238.48 96.76) (end 236.56 96.76) (width 1.27) (layer B.Cu) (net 25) (status 20))
 (segment (start 239.23 95.89) (end 239.23 96.01) (width 1.27) (layer B.Cu) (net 25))
 (segment (start 246.38 83.4) (end 246.38 84.821802) (width 1.27) (layer B.Cu) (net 25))
 (segment (start 244.118198 84.821802) (end 242.14 86.8) (width 1.27) (layer B.Cu) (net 25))
 (segment (start 242.14 86.8) (end 242.14 87.97) (width 1.27) (layer B.Cu) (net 25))
 (segment (start 239.23 96.01) (end 238.48 96.76) (width 1.27) (layer B.Cu) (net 25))
 (segment (start 239.99 90.12) (end 239.99 95.13) (width 1.27) (layer B.Cu) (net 25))
 (segment (start 242.14 87.97) (end 239.99 90.12) (width 1.27) (layer B.Cu) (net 25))
 (segment (start 236.56 96.76) (end 236.19 96.76) (width 1.27) (layer B.Cu) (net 25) (status 30))
 (segment (start 243.84 100.33) (end 243.55 100.33) (width 1.27) (layer B.Cu) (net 25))
 (segment (start 243.55 100.33) (end 239.23 96.01) (width 1.27) (layer B.Cu) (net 25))
 (segment (start 255.27 102.87) (end 246.38 102.87) (width 1.27) (layer B.Cu) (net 25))
 (segment (start 246.38 102.87) (end 243.84 100.33) (width 1.27) (layer B.Cu) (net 25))
 (segment (start 257.81 107.95) (end 257.81 105.41) (width 1.27) (layer B.Cu) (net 25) (status 10))
 (segment (start 257.81 105.41) (end 255.27 102.87) (width 1.27) (layer B.Cu) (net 25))
 (segment (start 235.18 94.22) (end 236.56 94.22) (width 1.27) (layer B.Cu) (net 26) (status 20))
 (segment (start 233.94 95.46) (end 235.18 94.22) (width 1.27) (layer B.Cu) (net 26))
 (segment (start 229.41 94.48) (end 230.39 95.46) (width 1.27) (layer B.Cu) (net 26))
 (segment (start 229.41 83.13) (end 229.41 94.48) (width 1.27) (layer B.Cu) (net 26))
 (segment (start 229.03001 82.75001) (end 229.41 83.13) (width 1.27) (layer B.Cu) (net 26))
 (segment (start 228.80001 82.75001) (end 229.03001 82.75001) (width 1.27) (layer B.Cu) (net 26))
 (segment (start 241.3 62.162081) (end 237.422081 66.04) (width 1.27) (layer B.Cu) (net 26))
 (segment (start 230.39 95.46) (end 233.94 95.46) (width 1.27) (layer B.Cu) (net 26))
 (segment (start 237.422081 66.04) (end 227.33 66.04) (width 1.27) (layer B.Cu) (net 26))
 (segment (start 227.33 66.04) (end 223.52 69.85) (width 1.27) (layer B.Cu) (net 26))
 (segment (start 241.3 60.96) (end 241.3 62.162081) (width 1.27) (layer B.Cu) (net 26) (status 10))
 (segment (start 223.52 69.85) (end 223.52 77.47) (width 1.27) (layer B.Cu) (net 26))
 (segment (start 223.52 77.47) (end 228.80001 82.75001) (width 1.27) (layer B.Cu) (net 26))
 (segment (start 214.63 101.6) (end 219.71 101.6) (width 1.27) (layer B.Cu) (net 22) (status 30))
 (segment (start 219.71 101.6) (end 220.912081 101.6) (width 1.27) (layer B.Cu) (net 22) (status 10))
 (segment (start 223.49 101.6) (end 220.912081 101.6) (width 1.27) (layer B.Cu) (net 22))
 (segment (start 225.87 103.98) (end 223.49 101.6) (width 1.27) (layer B.Cu) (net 22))
 (segment (start 225.9 103.98) (end 225.87 103.98) (width 1.27) (layer B.Cu) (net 22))
 (segment (start 229.87 107.95) (end 225.9 103.98) (width 1.27) (layer B.Cu) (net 22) (status 10))
 (segment (start 219.71 78.74) (end 214.63 78.74) (width 1.27) (layer B.Cu) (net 14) (status 30))
 (segment (start 220.912081 78.74) (end 221.092081 78.92) (width 1.27) (layer B.Cu) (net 14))
 (segment (start 219.71 78.74) (end 220.912081 78.74) (width 1.27) (layer B.Cu) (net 14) (status 10))
 (segment (start 221.092081 78.92) (end 221.89 78.92) (width 1.27) (layer B.Cu) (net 14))
 (segment (start 226.26001 83.29001) (end 226.31001 83.29001) (width 1.27) (layer B.Cu) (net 14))
 (segment (start 221.89 78.92) (end 226.26001 83.29001) (width 1.27) (layer B.Cu) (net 14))
 (segment (start 226.31001 83.29001) (end 227.12 84.1) (width 1.27) (layer B.Cu) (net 14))
 (segment (start 234.95 106.68) (end 234.95 107.95) (width 1.27) (layer B.Cu) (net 14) (status 20))
 (segment (start 227.12 84.1) (end 227.12 96.31) (width 1.27) (layer B.Cu) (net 14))
 (segment (start 234.95 106.747919) (end 234.95 107.95) (width 1.27) (layer B.Cu) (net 14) (status 20))
 (segment (start 234.95 104.14) (end 234.95 106.747919) (width 1.27) (layer B.Cu) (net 14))
 (segment (start 227.12 96.31) (end 234.95 104.14) (width 1.27) (layer B.Cu) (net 14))
 (segment (start 214.63 81.28) (end 219.71 81.28) (width 1.27) (layer B.Cu) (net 15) (status 30))
 (via (at 224.67 99.14) (size 1.778) (drill 0.889) (layers F.Cu B.Cu) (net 15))
 (segment (start 224.67 86.286198) (end 224.67 99.14) (width 1.27) (layer B.Cu) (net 15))
 (segment (start 219.71 81.28) (end 224.67 86.24) (width 1.27) (layer B.Cu) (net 15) (status 10))
 (segment (start 224.67 86.24) (end 224.67 86.286198) (width 1.27) (layer B.Cu) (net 15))
 (segment (start 237.49 107.95) (end 237.49 109.22) (width 1.27) (layer B.Cu) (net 15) (status 10))
 (segment (start 237.49 109.22) (end 236.22 110.49) (width 1.27) (layer B.Cu) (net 15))
 (segment (start 236.22 110.49) (end 227.33 110.49) (width 1.27) (layer B.Cu) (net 15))
 (segment (start 227.33 110.49) (end 224.79 107.95) (width 1.27) (layer B.Cu) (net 15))
 (segment (start 224.79 107.95) (end 223.52 106.68) (width 1.27) (layer B.Cu) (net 15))
 (via (at 223.52 105.41) (size 1.778) (drill 0.889) (layers F.Cu B.Cu) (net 15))
 (segment (start 223.52 106.68) (end 223.52 105.41) (width 1.27) (layer B.Cu) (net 15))
 (segment (start 219.71 68.58) (end 214.63 68.58) (width 1.27) (layer B.Cu) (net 10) (status 30))
 (segment (start 214.63 71.12) (end 219.71 71.12) (width 1.27) (layer B.Cu) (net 11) (status 30))
 (segment (start 219.71 73.66) (end 214.63 73.66) (width 1.27) (layer B.Cu) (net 12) (status 30))
 (segment (start 214.63 76.2) (end 219.71 76.2) (width 1.27) (layer B.Cu) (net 13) (status 30))
 (segment (start 255.27 99.06) (end 254 99.06) (width 1.27) (layer B.Cu) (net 13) (status 20))
 (segment (start 260.35 104.14) (end 255.27 99.06) (width 1.27) (layer B.Cu) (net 13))
 (segment (start 260.35 109.22) (end 260.35 104.14) (width 1.27) (layer B.Cu) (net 13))
 (segment (start 219.71 110.681522) (end 221.865957 112.837479) (width 1.27) (layer B.Cu) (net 13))
 (segment (start 256.732521 112.837479) (end 260.35 109.22) (width 1.27) (layer B.Cu) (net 13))
 (segment (start 213.36 76.2) (end 210.82 78.74) (width 1.27) (layer B.Cu) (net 13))
 (segment (start 210.82 78.74) (end 210.82 109.22) (width 1.27) (layer B.Cu) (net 13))
 (segment (start 210.82 109.22) (end 212.09 110.49) (width 1.27) (layer B.Cu) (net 13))
 (segment (start 221.865957 112.837479) (end 256.732521 112.837479) (width 1.27) (layer B.Cu) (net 13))
 (segment (start 212.09 110.49) (end 219.71 110.49) (width 1.27) (layer B.Cu) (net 13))
 (segment (start 214.63 76.2) (end 213.36 76.2) (width 1.27) (layer B.Cu) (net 13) (status 10))
 (segment (start 219.71 110.49) (end 219.71 110.681522) (width 1.27) (layer B.Cu) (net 13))
 (segment (start 219.71 83.82) (end 214.63 83.82) (width 1.27) (layer B.Cu) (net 16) (status 30))
 (segment (start 214.63 86.36) (end 219.71 86.36) (width 1.27) (layer B.Cu) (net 17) (status 30))
 (segment (start 219.71 88.9) (end 214.63 88.9) (width 1.27) (layer B.Cu) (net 18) (status 30))
 (segment (start 219.71 93.98) (end 214.63 93.98) (width 1.27) (layer B.Cu) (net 19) (status 30))
 (segment (start 214.63 96.52) (end 219.71 96.52) (width 1.27) (layer B.Cu) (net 20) (status 30))
 (segment (start 219.71 99.06) (end 214.63 99.06) (width 1.27) (layer B.Cu) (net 21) (status 30))
 (segment (start 219.71 104.14) (end 214.63 104.14) (width 1.27) (layer B.Cu) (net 23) (status 30))
 (segment (start 214.63 106.68) (end 219.71 106.68) (width 1.27) (layer B.Cu) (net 24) (status 30))
 (via (at 219.075 113.665) (size 1.778) (drill 0.889) (layers F.Cu B.Cu) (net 24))
 (segment (start 219.71 106.68) (end 219.71 106.72) (width 1.27) (layer B.Cu) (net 24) (status 30))
 (via (at 223.52 110.04) (size 1.778) (drill 0.889) (layers F.Cu B.Cu) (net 24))
 (segment (start 220.16 106.68) (end 223.52 110.04) (width 1.27) (layer B.Cu) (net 24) (status 10))
 (segment (start 219.71 106.68) (end 220.16 106.68) (width 1.27) (layer B.Cu) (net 24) (status 30))
 (segment (start 220.98 115.57) (end 219.075 113.665) (width 1.27) (layer B.Cu) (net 24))
 (segment (start 259.08 115.57) (end 220.98 115.57) (width 1.27) (layer B.Cu) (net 24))
 (segment (start 262.89 102.87) (end 262.89 111.76) (width 1.27) (layer B.Cu) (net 24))
 (segment (start 256.54 63.432081) (end 259.08 65.972081) (width 1.27) (layer B.Cu) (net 24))
 (segment (start 262.89 111.76) (end 259.08 115.57) (width 1.27) (layer B.Cu) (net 24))
 (segment (start 256.54 60.96) (end 256.54 63.432081) (width 1.27) (layer B.Cu) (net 24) (status 10))
 (segment (start 260.985 100.965) (end 262.89 102.87) (width 1.27) (layer B.Cu) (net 24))
 (segment (start 259.08 99.695) (end 260.35 100.965) (width 1.27) (layer B.Cu) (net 24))
 (segment (start 259.08 65.972081) (end 259.08 99.695) (width 1.27) (layer B.Cu) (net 24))
 (segment (start 260.35 100.965) (end 260.985 100.965) (width 1.27) (layer B.Cu) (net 24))
 (segment (start 235.118 87.97) (end 235.712 87.376) (width 1.27) (layer B.Cu) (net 5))
 (segment (start 231.59 87.97) (end 235.118 87.97) (width 1.27) (layer B.Cu) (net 5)))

